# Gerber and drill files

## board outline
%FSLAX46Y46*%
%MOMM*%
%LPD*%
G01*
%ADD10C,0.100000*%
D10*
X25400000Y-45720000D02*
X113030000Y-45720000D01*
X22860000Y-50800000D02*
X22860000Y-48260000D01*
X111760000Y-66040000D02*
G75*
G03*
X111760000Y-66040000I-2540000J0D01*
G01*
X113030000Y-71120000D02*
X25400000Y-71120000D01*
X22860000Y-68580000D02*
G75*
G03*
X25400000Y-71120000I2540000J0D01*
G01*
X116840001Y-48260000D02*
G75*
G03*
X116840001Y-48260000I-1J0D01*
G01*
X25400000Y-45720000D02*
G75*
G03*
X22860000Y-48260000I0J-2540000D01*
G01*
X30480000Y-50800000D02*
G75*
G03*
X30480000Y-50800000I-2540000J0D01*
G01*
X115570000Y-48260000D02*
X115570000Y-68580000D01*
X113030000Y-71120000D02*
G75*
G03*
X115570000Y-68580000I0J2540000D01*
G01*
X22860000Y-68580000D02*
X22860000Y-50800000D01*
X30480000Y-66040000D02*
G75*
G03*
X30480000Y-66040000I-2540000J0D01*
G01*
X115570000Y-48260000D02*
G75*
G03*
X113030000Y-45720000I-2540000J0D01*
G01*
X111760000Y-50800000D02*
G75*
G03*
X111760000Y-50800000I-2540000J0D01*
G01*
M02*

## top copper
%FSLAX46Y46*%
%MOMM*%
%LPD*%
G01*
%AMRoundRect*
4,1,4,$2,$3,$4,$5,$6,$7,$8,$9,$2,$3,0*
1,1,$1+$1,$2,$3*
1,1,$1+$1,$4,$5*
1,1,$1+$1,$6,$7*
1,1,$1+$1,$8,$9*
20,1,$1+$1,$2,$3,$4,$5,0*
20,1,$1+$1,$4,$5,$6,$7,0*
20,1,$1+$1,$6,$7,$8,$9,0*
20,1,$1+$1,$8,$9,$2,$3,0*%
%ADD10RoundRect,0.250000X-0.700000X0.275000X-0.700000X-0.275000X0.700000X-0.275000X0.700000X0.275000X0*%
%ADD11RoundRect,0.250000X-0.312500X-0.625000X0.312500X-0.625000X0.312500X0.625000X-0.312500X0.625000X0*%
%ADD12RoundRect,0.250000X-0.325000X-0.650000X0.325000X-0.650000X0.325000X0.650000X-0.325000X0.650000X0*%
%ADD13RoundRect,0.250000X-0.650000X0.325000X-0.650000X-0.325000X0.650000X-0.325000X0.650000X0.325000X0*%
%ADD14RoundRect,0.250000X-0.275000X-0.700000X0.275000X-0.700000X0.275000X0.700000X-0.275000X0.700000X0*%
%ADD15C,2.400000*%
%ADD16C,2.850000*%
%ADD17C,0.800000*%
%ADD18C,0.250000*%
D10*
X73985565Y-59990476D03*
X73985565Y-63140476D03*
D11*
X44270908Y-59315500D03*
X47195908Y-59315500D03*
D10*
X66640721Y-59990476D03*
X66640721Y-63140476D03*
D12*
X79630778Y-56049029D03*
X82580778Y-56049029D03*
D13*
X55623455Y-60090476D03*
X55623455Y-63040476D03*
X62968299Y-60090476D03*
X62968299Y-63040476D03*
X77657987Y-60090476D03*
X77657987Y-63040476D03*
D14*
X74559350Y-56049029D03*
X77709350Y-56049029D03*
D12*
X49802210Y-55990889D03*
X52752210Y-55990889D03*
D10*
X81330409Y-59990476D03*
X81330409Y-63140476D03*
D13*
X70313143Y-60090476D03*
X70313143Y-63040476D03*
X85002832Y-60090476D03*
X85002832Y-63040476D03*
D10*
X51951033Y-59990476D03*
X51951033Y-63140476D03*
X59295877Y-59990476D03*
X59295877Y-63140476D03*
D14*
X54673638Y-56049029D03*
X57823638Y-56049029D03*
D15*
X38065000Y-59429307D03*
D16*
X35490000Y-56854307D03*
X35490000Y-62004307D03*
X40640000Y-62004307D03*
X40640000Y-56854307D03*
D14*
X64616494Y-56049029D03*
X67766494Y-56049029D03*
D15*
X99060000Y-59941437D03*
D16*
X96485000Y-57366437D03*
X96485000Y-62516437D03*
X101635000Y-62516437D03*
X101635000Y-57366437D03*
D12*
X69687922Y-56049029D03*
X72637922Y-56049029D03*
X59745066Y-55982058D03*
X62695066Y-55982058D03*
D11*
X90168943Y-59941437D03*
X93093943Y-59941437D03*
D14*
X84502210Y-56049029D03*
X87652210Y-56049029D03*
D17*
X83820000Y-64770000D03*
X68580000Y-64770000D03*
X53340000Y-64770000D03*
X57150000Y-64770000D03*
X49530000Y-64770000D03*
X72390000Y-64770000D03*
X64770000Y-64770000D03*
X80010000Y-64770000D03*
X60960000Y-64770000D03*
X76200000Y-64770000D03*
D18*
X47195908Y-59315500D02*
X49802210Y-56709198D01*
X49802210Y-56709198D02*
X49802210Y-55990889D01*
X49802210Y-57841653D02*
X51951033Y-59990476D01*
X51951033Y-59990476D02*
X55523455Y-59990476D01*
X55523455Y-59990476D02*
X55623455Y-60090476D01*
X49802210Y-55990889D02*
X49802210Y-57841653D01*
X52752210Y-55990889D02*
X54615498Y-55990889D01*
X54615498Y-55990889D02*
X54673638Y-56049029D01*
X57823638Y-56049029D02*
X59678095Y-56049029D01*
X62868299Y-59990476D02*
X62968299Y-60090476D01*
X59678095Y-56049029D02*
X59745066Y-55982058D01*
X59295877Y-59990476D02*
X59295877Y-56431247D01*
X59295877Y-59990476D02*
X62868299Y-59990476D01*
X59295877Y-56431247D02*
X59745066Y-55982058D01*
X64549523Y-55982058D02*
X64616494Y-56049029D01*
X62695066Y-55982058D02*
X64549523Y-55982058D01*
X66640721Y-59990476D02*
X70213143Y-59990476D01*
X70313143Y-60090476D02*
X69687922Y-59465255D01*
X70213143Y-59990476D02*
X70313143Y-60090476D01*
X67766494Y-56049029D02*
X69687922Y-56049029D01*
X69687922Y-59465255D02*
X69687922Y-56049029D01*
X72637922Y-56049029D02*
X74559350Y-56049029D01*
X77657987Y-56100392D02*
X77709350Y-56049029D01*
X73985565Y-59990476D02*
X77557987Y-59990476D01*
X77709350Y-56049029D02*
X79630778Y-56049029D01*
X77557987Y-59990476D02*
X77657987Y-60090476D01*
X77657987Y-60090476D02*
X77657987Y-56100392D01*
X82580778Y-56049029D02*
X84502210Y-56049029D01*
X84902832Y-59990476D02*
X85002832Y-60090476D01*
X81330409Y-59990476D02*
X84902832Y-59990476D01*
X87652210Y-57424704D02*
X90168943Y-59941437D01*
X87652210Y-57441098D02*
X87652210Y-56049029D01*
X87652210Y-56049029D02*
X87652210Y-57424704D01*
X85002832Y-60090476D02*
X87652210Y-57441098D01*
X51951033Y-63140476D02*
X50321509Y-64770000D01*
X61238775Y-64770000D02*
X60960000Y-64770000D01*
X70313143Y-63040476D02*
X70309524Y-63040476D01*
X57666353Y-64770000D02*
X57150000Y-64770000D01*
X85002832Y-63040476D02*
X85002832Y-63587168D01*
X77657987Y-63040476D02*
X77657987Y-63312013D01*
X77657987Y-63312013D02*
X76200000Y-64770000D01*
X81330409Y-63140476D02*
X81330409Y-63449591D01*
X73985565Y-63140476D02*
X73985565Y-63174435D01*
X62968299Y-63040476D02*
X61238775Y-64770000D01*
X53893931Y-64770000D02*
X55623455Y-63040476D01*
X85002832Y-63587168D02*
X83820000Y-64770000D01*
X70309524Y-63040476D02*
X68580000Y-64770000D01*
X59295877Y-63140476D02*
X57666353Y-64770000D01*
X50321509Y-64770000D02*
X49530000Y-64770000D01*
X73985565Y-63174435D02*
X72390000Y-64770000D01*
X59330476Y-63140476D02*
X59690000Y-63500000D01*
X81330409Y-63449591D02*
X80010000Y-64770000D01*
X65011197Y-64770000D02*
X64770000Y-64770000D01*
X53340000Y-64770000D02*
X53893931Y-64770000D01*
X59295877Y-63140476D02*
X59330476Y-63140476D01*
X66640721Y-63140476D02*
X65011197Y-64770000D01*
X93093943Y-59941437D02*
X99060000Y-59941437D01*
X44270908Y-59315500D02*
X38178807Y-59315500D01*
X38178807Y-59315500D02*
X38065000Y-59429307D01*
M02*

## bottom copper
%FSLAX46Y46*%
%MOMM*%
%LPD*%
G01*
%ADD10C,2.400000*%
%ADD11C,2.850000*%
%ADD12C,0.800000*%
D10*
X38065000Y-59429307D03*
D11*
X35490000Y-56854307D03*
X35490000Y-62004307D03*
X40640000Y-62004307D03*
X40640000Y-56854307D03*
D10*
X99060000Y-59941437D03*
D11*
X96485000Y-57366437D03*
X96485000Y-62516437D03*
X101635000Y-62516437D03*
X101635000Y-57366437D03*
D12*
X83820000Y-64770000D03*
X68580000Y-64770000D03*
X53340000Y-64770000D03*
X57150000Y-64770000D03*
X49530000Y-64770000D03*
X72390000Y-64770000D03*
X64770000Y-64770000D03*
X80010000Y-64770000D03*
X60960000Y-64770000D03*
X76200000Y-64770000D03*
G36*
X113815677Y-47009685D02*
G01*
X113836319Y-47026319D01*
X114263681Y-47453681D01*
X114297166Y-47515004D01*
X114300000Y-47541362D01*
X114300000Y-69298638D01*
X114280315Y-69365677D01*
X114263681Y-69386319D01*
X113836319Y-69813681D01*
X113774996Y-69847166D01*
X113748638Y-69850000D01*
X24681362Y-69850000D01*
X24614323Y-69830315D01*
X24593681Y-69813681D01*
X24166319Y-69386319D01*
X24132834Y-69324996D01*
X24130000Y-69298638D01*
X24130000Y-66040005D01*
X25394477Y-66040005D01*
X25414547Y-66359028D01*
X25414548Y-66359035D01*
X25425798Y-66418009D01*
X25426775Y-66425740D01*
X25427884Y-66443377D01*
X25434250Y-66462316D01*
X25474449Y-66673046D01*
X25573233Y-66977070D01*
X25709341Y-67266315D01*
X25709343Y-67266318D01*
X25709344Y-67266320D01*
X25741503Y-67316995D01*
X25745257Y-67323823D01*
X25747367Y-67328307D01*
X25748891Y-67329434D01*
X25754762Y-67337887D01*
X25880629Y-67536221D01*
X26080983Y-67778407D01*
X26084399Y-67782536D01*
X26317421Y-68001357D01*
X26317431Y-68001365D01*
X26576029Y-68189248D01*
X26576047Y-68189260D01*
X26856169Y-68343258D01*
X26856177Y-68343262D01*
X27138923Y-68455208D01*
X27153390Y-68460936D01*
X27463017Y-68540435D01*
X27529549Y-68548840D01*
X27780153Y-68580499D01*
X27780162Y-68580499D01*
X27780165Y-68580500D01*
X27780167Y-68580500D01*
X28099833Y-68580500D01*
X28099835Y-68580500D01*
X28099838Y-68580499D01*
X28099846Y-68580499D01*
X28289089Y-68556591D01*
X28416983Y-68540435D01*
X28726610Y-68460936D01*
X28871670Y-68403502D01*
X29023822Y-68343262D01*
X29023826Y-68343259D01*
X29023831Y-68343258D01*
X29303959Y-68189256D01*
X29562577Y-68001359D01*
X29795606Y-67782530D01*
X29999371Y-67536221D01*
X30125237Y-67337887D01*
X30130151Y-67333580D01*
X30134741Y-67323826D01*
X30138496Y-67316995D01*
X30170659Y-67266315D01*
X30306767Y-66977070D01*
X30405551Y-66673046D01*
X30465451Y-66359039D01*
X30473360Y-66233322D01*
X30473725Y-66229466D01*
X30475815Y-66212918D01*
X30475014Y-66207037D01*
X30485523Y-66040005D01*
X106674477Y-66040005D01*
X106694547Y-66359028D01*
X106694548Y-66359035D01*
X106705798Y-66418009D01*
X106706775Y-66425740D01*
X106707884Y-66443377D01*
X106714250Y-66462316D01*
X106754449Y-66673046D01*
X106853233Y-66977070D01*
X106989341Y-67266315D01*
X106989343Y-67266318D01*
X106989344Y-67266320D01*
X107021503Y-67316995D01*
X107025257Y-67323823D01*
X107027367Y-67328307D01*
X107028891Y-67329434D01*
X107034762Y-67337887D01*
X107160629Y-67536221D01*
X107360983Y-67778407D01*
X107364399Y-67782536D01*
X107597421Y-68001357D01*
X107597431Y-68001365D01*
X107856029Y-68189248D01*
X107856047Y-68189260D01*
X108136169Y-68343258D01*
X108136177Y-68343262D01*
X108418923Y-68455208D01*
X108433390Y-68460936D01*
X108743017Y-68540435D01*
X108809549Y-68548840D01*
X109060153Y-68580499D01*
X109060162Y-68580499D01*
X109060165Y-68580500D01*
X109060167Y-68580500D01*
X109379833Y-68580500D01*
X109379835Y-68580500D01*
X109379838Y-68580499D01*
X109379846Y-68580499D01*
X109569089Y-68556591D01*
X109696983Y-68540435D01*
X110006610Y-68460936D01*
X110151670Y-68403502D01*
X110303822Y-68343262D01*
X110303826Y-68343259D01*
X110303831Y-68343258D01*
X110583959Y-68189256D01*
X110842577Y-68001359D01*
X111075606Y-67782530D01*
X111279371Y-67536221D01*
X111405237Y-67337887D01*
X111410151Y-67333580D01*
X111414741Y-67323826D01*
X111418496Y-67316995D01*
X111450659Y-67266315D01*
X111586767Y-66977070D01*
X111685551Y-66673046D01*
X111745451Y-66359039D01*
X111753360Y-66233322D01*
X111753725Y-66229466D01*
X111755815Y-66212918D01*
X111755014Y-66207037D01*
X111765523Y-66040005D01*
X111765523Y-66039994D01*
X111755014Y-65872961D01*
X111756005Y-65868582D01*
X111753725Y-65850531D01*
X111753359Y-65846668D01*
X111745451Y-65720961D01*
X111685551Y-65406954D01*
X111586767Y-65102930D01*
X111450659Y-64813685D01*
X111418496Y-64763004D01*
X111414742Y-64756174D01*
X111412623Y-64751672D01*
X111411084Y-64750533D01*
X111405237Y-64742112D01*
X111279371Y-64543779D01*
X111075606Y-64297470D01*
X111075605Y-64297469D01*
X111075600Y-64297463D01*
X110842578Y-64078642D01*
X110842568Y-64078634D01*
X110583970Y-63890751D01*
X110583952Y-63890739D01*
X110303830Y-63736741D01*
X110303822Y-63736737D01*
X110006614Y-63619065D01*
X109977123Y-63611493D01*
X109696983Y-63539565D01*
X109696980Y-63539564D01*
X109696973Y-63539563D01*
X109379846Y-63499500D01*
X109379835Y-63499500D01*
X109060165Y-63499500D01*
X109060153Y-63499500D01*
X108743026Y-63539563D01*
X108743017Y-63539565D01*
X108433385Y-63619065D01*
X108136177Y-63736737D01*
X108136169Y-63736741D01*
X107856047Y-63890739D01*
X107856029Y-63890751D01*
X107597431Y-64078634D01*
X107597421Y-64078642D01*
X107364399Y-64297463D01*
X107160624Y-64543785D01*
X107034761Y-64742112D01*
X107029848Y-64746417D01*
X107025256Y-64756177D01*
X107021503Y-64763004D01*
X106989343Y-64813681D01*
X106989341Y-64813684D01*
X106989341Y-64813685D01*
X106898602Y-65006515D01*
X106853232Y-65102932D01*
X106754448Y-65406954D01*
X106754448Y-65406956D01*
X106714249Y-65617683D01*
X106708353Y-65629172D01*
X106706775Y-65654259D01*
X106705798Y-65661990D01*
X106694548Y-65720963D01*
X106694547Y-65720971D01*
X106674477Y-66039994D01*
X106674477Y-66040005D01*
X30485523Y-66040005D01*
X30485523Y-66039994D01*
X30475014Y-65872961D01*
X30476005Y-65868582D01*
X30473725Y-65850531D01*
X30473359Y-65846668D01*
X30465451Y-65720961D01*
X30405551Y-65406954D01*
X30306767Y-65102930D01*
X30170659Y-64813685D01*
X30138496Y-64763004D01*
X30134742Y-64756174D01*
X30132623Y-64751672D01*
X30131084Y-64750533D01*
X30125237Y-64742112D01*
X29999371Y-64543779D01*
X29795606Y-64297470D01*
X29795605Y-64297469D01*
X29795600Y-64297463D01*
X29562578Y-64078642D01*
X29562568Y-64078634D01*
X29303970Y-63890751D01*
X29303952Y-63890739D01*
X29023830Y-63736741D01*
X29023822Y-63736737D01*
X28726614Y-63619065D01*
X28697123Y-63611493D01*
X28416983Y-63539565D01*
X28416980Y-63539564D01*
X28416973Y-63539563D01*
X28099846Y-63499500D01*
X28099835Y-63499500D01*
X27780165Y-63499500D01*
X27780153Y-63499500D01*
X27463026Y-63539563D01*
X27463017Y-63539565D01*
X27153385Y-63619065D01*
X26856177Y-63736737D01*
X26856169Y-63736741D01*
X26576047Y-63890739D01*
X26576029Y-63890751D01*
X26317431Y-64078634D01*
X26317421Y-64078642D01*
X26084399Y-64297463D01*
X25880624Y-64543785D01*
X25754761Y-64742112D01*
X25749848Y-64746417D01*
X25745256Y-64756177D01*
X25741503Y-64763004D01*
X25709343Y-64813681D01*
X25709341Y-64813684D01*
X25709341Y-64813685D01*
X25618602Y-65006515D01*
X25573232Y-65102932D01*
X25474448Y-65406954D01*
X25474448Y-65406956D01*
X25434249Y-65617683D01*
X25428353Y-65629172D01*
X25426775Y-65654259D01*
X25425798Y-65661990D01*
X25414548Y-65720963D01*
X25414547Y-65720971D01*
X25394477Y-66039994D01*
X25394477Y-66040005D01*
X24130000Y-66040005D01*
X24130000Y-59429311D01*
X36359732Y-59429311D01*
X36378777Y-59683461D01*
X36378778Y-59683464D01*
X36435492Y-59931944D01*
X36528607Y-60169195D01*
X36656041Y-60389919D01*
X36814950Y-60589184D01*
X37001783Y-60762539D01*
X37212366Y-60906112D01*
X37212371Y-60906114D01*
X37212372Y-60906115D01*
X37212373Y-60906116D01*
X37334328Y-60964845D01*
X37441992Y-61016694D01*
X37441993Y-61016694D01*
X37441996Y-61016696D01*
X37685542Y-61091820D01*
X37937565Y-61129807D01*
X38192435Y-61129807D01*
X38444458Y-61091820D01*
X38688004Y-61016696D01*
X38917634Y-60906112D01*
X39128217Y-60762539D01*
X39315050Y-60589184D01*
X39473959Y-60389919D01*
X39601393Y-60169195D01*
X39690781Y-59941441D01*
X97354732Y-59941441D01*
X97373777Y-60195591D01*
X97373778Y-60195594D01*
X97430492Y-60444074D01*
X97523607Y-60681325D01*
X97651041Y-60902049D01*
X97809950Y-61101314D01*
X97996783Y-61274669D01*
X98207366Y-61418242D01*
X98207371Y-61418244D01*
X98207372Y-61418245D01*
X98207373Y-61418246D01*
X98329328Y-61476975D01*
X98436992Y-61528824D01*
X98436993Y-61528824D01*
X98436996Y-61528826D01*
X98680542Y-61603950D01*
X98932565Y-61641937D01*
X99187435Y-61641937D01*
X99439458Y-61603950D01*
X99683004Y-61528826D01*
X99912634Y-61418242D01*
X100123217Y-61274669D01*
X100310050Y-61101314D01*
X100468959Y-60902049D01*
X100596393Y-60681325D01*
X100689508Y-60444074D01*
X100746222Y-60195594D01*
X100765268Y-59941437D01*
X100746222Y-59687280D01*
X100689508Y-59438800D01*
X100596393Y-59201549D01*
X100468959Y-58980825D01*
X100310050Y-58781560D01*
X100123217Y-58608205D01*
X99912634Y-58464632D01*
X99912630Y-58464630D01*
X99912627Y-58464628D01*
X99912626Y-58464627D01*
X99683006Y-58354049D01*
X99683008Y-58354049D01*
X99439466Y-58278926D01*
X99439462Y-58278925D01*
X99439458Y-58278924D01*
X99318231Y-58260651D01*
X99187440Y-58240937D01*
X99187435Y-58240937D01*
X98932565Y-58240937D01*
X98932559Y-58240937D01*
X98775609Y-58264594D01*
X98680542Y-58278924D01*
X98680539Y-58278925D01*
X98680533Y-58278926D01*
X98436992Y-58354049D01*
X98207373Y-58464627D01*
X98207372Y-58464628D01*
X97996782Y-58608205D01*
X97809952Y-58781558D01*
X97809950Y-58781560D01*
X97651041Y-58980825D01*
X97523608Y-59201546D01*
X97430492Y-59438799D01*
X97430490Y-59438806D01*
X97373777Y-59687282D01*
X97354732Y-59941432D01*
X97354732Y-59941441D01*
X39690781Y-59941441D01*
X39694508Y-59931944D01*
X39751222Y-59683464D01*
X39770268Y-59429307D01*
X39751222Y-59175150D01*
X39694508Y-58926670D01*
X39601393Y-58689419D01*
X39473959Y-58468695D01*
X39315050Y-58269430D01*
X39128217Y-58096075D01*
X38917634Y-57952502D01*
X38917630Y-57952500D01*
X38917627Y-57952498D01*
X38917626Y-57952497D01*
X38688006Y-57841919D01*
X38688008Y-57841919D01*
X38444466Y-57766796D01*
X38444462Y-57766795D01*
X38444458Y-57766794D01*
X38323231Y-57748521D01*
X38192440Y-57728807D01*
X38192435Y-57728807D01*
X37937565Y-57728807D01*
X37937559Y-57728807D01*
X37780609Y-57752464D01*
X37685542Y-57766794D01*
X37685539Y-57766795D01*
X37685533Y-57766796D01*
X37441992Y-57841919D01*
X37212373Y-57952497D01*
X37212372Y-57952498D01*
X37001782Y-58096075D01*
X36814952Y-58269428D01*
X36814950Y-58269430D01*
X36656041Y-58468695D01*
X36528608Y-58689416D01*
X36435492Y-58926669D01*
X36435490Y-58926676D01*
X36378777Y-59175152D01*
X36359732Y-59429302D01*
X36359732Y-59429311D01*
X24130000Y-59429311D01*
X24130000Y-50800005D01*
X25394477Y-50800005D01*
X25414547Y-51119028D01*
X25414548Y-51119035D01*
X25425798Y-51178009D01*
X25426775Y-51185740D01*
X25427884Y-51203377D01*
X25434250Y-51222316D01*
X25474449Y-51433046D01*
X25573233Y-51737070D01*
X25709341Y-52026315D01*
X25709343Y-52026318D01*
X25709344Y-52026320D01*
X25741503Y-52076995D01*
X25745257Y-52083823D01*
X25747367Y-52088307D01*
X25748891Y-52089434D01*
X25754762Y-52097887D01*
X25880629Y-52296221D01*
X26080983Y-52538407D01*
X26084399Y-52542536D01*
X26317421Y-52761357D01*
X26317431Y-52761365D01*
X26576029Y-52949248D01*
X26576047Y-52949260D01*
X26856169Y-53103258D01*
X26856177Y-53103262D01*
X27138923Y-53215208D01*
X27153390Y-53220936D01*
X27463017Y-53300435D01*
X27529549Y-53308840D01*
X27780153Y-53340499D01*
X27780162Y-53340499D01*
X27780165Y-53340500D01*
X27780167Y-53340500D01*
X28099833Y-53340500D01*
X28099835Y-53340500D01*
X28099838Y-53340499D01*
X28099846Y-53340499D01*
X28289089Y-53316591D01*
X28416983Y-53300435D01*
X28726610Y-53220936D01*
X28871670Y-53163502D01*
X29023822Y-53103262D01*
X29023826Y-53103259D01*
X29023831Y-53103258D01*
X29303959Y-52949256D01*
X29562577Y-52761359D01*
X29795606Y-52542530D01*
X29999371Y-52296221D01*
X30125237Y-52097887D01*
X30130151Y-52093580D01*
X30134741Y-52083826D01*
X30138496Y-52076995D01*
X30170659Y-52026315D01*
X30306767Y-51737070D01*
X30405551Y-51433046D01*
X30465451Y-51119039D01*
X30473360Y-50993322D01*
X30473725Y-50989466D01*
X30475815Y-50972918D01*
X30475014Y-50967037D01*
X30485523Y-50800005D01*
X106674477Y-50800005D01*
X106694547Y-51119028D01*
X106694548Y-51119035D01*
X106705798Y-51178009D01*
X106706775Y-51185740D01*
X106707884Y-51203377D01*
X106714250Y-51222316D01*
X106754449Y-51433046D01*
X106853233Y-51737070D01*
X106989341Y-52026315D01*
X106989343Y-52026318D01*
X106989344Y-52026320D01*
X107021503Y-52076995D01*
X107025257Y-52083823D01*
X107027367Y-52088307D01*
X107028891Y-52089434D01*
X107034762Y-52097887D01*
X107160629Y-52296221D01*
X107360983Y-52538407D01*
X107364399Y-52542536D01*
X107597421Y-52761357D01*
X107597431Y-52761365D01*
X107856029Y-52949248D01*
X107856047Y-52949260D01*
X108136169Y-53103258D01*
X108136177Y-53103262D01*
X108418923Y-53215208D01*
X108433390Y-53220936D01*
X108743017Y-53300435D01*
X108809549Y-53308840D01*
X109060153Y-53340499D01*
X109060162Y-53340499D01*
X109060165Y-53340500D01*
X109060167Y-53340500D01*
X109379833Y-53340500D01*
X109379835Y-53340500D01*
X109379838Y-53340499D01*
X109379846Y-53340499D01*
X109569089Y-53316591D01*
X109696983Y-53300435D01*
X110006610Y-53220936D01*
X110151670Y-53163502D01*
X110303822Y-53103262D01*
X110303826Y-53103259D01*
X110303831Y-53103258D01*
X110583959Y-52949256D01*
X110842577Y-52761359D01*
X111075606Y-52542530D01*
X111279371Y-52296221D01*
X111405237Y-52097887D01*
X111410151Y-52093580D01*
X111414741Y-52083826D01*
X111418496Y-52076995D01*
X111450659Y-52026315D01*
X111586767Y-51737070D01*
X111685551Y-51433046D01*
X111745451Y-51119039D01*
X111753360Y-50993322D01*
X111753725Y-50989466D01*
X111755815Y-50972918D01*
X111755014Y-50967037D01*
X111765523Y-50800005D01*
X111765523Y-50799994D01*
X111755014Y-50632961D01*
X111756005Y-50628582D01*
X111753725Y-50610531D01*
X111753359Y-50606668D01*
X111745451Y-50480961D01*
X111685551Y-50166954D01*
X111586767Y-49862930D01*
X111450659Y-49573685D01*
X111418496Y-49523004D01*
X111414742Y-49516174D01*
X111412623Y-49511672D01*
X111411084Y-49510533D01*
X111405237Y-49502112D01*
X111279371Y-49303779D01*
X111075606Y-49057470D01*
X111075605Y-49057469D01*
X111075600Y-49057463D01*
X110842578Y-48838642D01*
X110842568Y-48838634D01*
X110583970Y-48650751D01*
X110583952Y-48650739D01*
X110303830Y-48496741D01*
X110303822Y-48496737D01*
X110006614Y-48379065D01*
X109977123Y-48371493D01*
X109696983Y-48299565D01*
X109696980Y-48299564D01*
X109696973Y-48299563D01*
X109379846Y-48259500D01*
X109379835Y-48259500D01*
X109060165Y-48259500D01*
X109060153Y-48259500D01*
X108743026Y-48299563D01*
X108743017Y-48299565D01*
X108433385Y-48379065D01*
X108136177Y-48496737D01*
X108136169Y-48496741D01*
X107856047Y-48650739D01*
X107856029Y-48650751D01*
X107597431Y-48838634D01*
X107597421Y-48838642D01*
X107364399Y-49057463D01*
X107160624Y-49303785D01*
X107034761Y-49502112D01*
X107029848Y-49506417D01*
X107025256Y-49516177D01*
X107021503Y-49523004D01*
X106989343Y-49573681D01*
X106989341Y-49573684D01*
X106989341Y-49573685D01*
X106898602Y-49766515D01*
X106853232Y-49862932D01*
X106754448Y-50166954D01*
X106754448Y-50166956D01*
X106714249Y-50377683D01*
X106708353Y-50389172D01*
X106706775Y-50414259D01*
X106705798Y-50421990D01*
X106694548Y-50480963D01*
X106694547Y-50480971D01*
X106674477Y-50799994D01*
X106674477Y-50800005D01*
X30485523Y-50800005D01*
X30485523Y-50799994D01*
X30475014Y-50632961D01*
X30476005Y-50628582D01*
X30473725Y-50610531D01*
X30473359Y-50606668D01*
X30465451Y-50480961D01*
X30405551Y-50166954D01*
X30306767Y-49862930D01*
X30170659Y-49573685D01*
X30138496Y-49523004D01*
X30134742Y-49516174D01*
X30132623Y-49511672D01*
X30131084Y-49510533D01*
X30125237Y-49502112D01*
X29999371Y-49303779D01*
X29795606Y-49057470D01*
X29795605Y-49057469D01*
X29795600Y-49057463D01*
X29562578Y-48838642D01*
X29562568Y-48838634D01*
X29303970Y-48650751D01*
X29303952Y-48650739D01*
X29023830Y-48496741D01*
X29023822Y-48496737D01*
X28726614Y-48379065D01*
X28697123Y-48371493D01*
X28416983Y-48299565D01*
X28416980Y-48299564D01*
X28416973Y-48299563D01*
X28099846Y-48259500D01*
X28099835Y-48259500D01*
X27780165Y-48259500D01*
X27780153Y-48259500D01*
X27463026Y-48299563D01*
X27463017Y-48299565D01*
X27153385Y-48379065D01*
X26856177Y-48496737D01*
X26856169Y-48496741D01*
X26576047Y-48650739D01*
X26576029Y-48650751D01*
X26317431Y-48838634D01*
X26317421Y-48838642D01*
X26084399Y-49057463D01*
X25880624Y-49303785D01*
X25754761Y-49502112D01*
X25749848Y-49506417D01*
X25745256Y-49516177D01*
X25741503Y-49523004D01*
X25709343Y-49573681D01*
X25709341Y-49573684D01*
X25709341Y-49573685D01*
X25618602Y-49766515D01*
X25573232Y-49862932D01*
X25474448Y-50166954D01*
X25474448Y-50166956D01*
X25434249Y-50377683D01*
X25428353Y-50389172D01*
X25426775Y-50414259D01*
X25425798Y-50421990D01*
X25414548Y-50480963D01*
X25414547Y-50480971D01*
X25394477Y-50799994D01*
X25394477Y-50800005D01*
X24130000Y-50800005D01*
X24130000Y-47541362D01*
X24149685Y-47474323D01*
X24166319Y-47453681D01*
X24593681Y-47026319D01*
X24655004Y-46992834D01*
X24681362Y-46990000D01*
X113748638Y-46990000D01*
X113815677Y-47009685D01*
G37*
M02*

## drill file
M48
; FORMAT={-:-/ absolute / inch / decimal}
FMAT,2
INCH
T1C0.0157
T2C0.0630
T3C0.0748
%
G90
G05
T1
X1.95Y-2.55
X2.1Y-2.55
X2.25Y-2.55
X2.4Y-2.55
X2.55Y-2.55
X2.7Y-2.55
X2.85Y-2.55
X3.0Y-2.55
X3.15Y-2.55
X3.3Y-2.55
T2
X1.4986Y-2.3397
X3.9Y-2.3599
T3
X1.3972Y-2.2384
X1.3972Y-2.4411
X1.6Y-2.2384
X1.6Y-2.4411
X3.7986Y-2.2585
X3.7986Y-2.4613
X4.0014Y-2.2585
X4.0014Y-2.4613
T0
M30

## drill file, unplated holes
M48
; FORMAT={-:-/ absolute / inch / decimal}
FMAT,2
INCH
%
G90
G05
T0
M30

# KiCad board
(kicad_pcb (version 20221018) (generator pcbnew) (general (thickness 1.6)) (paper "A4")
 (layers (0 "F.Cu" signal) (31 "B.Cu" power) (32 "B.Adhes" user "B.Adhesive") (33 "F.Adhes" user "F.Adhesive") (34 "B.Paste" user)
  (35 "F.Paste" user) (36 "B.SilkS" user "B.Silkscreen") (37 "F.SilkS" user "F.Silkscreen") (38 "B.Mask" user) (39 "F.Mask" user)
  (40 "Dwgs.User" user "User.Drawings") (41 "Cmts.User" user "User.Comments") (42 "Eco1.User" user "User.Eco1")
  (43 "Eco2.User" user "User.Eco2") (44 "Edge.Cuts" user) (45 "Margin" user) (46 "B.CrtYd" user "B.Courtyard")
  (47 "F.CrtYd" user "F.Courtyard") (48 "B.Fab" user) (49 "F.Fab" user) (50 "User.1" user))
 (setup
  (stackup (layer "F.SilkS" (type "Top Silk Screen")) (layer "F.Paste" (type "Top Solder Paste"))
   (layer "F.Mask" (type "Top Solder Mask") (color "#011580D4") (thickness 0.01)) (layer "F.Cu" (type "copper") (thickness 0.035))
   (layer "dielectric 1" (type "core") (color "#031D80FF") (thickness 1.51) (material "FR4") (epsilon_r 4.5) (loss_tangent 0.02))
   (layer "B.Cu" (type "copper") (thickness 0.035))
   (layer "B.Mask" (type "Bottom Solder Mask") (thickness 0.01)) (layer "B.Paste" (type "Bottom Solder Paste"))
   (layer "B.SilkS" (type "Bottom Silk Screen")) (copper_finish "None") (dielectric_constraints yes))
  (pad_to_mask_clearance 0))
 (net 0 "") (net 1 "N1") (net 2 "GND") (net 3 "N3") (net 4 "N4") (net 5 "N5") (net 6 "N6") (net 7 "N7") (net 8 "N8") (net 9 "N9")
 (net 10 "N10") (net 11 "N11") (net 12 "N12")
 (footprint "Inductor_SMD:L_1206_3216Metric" (layer "F.Cu") (at 73.985565 61.565476 -90)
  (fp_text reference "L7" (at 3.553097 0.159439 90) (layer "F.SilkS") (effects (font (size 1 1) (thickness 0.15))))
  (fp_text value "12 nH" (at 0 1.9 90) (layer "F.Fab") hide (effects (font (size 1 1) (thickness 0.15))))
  (pad "1" smd roundrect (at -1.575 0 270) (size 1.05 1.9) (layers "F.Cu" "F.Paste" "F.Mask") (roundrect_rratio 0.2380952381) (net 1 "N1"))
  (pad "2" smd roundrect (at 1.575 0 270) (size 1.05 1.9) (layers "F.Cu" "F.Paste" "F.Mask") (roundrect_rratio 0.2380952381) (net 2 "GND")))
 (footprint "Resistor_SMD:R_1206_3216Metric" (layer "F.Cu") (at 45.733408 59.3155)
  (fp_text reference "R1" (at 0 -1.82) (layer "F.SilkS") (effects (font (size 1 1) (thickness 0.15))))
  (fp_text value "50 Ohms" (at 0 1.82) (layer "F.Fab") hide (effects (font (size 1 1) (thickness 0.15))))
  (pad "1" smd roundrect (at -1.4625 0) (size 1.125 1.75) (layers "F.Cu" "F.Paste" "F.Mask") (roundrect_rratio 0.2222222222) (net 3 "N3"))
  (pad "2" smd roundrect (at 1.4625 0) (size 1.125 1.75) (layers "F.Cu" "F.Paste" "F.Mask") (roundrect_rratio 0.2222222222) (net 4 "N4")))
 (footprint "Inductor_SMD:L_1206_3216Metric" (layer "F.Cu") (at 66.640721 61.565476 -90)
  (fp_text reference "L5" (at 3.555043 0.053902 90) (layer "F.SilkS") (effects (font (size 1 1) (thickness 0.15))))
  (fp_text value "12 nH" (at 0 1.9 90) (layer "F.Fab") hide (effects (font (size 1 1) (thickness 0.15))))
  (pad "1" smd roundrect (at -1.575 0 270) (size 1.05 1.9) (layers "F.Cu" "F.Paste" "F.Mask") (roundrect_rratio 0.2380952381) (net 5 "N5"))
  (pad "2" smd roundrect (at 1.575 0 270) (size 1.05 1.9) (layers "F.Cu" "F.Paste" "F.Mask") (roundrect_rratio 0.2380952381) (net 2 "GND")))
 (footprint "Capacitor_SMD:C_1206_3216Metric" (layer "F.Cu") (at 81.105778 56.049029)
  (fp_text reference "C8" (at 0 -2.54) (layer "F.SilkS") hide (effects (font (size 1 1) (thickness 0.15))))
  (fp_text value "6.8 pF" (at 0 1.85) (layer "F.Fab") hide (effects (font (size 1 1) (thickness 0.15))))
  (pad "1" smd roundrect (at -1.475 0) (size 1.15 1.8) (layers "F.Cu" "F.Paste" "F.Mask") (roundrect_rratio 0.2173913043) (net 1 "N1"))
  (pad "2" smd roundrect (at 1.475 0) (size 1.15 1.8) (layers "F.Cu" "F.Paste" "F.Mask") (roundrect_rratio 0.2173913043) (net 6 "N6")))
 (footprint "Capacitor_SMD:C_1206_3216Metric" (layer "F.Cu") (at 55.623455 61.565476 -90)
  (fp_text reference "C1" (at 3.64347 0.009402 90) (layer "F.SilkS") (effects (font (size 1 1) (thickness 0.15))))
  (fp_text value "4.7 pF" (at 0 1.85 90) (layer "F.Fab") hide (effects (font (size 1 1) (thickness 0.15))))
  (pad "1" smd roundrect (at -1.475 0 270) (size 1.15 1.8) (layers "F.Cu" "F.Paste" "F.Mask") (roundrect_rratio 0.2173913043) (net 4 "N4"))
  (pad "2" smd roundrect (at 1.475 0 270) (size 1.15 1.8) (layers "F.Cu" "F.Paste" "F.Mask") (roundrect_rratio 0.2173913043) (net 2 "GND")))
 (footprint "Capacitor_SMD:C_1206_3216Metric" (layer "F.Cu") (at 62.968299 61.565476 -90)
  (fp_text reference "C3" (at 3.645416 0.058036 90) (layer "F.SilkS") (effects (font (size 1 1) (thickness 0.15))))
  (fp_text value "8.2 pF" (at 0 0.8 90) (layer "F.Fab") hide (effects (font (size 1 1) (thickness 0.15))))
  (pad "1" smd roundrect (at -1.475 0 270) (size 1.15 1.8) (layers "F.Cu" "F.Paste" "F.Mask") (roundrect_rratio 0.2173913043) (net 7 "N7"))
  (pad "2" smd roundrect (at 1.475 0 270) (size 1.15 1.8) (layers "F.Cu" "F.Paste" "F.Mask") (roundrect_rratio 0.2173913043) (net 2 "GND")))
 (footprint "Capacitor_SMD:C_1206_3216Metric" (layer "F.Cu") (at 77.657987 61.565476 -90)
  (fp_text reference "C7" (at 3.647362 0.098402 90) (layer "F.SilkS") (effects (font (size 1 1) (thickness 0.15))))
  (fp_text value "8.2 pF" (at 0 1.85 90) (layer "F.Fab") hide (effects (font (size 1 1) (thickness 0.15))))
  (pad "1" smd roundrect (at -1.475 0 270) (size 1.15 1.8) (layers "F.Cu" "F.Paste" "F.Mask") (roundrect_rratio 0.2173913043) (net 1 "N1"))
  (pad "2" smd roundrect (at 1.475 0 270) (size 1.15 1.8) (layers "F.Cu" "F.Paste" "F.Mask") (roundrect_rratio 0.2173913043) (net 2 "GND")))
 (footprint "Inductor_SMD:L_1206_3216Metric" (layer "F.Cu") (at 76.13435 56.049029)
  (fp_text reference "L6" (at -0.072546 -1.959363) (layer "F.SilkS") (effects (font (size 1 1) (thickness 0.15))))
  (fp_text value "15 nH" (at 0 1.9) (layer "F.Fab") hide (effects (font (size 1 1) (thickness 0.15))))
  (pad "1" smd roundrect (at -1.575 0) (size 1.05 1.9) (layers "F.Cu" "F.Paste" "F.Mask") (roundrect_rratio 0.2380952381) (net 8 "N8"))
  (pad "2" smd roundrect (at 1.575 0) (size 1.05 1.9) (layers "F.Cu" "F.Paste" "F.Mask") (roundrect_rratio 0.2380952381) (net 1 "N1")))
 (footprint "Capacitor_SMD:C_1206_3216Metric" (layer "F.Cu") (at 51.27721 55.990889)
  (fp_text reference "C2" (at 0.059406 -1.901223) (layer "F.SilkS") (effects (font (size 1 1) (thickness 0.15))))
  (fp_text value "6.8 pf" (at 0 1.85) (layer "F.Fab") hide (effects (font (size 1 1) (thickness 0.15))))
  (pad "1" smd roundrect (at -1.475 0) (size 1.15 1.8) (layers "F.Cu" "F.Paste" "F.Mask") (roundrect_rratio 0.2173913043) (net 4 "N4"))
  (pad "2" smd roundrect (at 1.475 0) (size 1.15 1.8) (layers "F.Cu" "F.Paste" "F.Mask") (roundrect_rratio 0.2173913043) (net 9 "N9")))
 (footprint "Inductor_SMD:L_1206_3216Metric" (layer "F.Cu") (at 81.330409 61.565476 -90)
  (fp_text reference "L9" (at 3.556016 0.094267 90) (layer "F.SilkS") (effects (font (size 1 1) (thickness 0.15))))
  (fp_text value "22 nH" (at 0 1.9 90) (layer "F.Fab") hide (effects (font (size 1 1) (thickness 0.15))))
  (pad "1" smd roundrect (at -1.575 0 270) (size 1.05 1.9) (layers "F.Cu" "F.Paste" "F.Mask") (roundrect_rratio 0.2380952381) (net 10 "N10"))
  (pad "2" smd roundrect (at 1.575 0 270) (size 1.05 1.9) (layers "F.Cu" "F.Paste" "F.Mask") (roundrect_rratio 0.2380952381) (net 2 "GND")))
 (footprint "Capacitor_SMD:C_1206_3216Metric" (layer "F.Cu") (at 70.313143 61.565476 -90)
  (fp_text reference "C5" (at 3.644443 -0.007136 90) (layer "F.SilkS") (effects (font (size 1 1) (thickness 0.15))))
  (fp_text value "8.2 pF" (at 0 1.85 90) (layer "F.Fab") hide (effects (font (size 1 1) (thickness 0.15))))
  (pad "1" smd roundrect (at -1.475 0 270) (size 1.15 1.8) (layers "F.Cu" "F.Paste" "F.Mask") (roundrect_rratio 0.2173913043) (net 5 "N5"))
  (pad "2" smd roundrect (at 1.475 0 270) (size 1.15 1.8) (layers "F.Cu" "F.Paste" "F.Mask") (roundrect_rratio 0.2173913043) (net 2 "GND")))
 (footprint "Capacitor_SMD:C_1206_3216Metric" (layer "F.Cu") (at 85.002832 61.565476 -90)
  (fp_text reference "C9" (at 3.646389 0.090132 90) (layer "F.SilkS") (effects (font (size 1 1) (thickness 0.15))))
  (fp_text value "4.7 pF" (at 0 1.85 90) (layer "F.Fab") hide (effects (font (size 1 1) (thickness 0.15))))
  (pad "1" smd roundrect (at -1.475 0 270) (size 1.15 1.8) (layers "F.Cu" "F.Paste" "F.Mask") (roundrect_rratio 0.2173913043) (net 10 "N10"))
  (pad "2" smd roundrect (at 1.475 0 270) (size 1.15 1.8) (layers "F.Cu" "F.Paste" "F.Mask") (roundrect_rratio 0.2173913043) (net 2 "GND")))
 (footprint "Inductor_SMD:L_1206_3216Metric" (layer "F.Cu") (at 51.951033 61.565476 -90)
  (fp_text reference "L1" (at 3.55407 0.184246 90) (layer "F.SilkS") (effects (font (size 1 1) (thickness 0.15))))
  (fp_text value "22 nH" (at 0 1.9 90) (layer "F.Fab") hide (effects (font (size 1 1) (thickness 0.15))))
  (pad "1" smd roundrect (at -1.575 0 270) (size 1.05 1.9) (layers "F.Cu" "F.Paste" "F.Mask") (roundrect_rratio 0.2380952381) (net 4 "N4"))
  (pad "2" smd roundrect (at 1.575 0 270) (size 1.05 1.9) (layers "F.Cu" "F.Paste" "F.Mask") (roundrect_rratio 0.2380952381) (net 2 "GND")))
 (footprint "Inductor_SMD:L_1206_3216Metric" (layer "F.Cu") (at 59.295877 61.565476 -90)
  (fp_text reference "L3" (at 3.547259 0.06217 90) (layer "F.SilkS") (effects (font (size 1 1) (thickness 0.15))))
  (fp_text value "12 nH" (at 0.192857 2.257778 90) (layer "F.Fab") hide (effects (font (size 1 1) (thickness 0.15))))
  (pad "1" smd roundrect (at -1.575 0 270) (size 1.05 1.9) (layers "F.Cu" "F.Paste" "F.Mask") (roundrect_rratio 0.2380952381) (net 7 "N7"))
  (pad "2" smd roundrect (at 1.575 0 270) (size 1.05 1.9) (layers "F.Cu" "F.Paste" "F.Mask") (roundrect_rratio 0.2380952381) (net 2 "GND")))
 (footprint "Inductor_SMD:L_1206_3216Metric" (layer "F.Cu") (at 56.248638 56.049029)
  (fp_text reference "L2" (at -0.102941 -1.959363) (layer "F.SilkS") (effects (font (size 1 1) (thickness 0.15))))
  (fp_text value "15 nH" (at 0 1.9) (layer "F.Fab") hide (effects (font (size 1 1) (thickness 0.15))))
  (pad "1" smd roundrect (at -1.575 0) (size 1.05 1.9) (layers "F.Cu" "F.Paste" "F.Mask") (roundrect_rratio 0.2380952381) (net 9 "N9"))
  (pad "2" smd roundrect (at 1.575 0) (size 1.05 1.9) (layers "F.Cu" "F.Paste" "F.Mask") (roundrect_rratio 0.2380952381) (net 7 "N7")))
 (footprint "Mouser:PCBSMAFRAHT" (layer "F.Cu") (at 38.065 59.429307)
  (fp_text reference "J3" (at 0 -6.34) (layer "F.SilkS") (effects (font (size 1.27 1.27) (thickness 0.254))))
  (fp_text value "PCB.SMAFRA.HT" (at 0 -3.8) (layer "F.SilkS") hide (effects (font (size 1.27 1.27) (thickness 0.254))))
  (pad "1" thru_hole circle (at 0 0) (size 2.4 2.4) (drill 1.6) (layers "*.Cu" "*.Mask") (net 3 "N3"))
  (pad "2" thru_hole circle (at -2.575 -2.575) (size 2.85 2.85) (drill 1.9) (layers "*.Cu" "*.Mask") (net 2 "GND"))
  (pad "3" thru_hole circle (at -2.575 2.575) (size 2.85 2.85) (drill 1.9) (layers "*.Cu" "*.Mask") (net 2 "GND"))
  (pad "4" thru_hole circle (at 2.575 2.575) (size 2.85 2.85) (drill 1.9) (layers "*.Cu" "*.Mask") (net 2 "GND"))
  (pad "5" thru_hole circle (at 2.575 -2.575) (size 2.85 2.85) (drill 1.9) (layers "*.Cu" "*.Mask") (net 2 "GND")))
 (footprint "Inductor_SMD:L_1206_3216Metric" (layer "F.Cu") (at 66.191494 56.049029)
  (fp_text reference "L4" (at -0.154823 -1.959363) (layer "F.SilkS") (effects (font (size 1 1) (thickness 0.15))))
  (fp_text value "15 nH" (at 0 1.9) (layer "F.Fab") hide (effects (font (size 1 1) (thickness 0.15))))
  (pad "1" smd roundrect (at -1.575 0) (size 1.05 1.9) (layers "F.Cu" "F.Paste" "F.Mask") (roundrect_rratio 0.2380952381) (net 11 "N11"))
  (pad "2" smd roundrect (at 1.575 0) (size 1.05 1.9) (layers "F.Cu" "F.Paste" "F.Mask") (roundrect_rratio 0.2380952381) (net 5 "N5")))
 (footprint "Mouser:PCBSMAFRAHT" (layer "F.Cu") (at 99.06 59.941437)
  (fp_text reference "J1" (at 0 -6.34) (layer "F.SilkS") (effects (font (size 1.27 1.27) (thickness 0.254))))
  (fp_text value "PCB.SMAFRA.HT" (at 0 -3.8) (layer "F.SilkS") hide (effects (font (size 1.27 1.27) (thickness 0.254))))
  (pad "1" thru_hole circle (at 0 0) (size 2.4 2.4) (drill 1.6) (layers "*.Cu" "*.Mask") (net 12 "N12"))
  (pad "2" thru_hole circle (at -2.575 -2.575) (size 2.85 2.85) (drill 1.9) (layers "*.Cu" "*.Mask") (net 2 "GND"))
  (pad "3" thru_hole circle (at -2.575 2.575) (size 2.85 2.85) (drill 1.9) (layers "*.Cu" "*.Mask") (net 2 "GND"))
  (pad "4" thru_hole circle (at 2.575 2.575) (size 2.85 2.85) (drill 1.9) (layers "*.Cu" "*.Mask") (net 2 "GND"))
  (pad "5" thru_hole circle (at 2.575 -2.575) (size 2.85 2.85) (drill 1.9) (layers "*.Cu" "*.Mask") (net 2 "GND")))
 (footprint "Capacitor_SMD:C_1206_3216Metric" (layer "F.Cu") (at 71.162922 56.049029)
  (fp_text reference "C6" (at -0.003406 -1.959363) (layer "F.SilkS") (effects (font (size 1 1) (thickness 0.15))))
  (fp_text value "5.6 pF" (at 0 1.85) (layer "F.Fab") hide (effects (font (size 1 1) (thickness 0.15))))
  (pad "1" smd roundrect (at -1.475 0) (size 1.15 1.8) (layers "F.Cu" "F.Paste" "F.Mask") (roundrect_rratio 0.2173913043) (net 5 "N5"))
  (pad "2" smd roundrect (at 1.475 0) (size 1.15 1.8) (layers "F.Cu" "F.Paste" "F.Mask") (roundrect_rratio 0.2173913043) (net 8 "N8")))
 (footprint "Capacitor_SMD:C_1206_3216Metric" (layer "F.Cu") (at 61.220066 55.982058)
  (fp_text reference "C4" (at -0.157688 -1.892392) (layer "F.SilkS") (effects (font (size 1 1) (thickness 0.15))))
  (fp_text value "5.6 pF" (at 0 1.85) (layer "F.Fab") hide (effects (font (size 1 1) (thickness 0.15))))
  (pad "1" smd roundrect (at -1.475 0) (size 1.15 1.8) (layers "F.Cu" "F.Paste" "F.Mask") (roundrect_rratio 0.2173913043) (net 7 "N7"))
  (pad "2" smd roundrect (at 1.475 0) (size 1.15 1.8) (layers "F.Cu" "F.Paste" "F.Mask") (roundrect_rratio 0.2173913043) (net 11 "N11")))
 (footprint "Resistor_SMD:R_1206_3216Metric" (layer "F.Cu") (at 91.631443 59.941437)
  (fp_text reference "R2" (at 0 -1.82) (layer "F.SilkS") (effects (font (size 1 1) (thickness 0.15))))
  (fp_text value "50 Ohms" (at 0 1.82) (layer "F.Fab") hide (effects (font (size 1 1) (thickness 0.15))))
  (pad "1" smd roundrect (at -1.4625 0) (size 1.125 1.75) (layers "F.Cu" "F.Paste" "F.Mask") (roundrect_rratio 0.2222222222) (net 10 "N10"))
  (pad "2" smd roundrect (at 1.4625 0) (size 1.125 1.75) (layers "F.Cu" "F.Paste" "F.Mask") (roundrect_rratio 0.2222222222) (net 12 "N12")))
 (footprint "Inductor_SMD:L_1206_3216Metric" (layer "F.Cu") (at 86.07721 56.049029)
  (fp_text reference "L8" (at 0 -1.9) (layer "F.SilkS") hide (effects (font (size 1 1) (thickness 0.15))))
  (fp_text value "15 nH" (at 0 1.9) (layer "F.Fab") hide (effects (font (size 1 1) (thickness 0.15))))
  (pad "1" smd roundrect (at -1.575 0) (size 1.05 1.9) (layers "F.Cu" "F.Paste" "F.Mask") (roundrect_rratio 0.2380952381) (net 6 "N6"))
  (pad "2" smd roundrect (at 1.575 0) (size 1.05 1.9) (layers "F.Cu" "F.Paste" "F.Mask") (roundrect_rratio 0.2380952381) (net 10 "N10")))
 (gr_line (start 25.4 45.72) (end 113.03 45.72) (stroke (width 0.1) (type default)) (layer "Edge.Cuts"))
 (gr_line (start 22.86 50.8) (end 22.86 48.26) (stroke (width 0.1) (type default)) (layer "Edge.Cuts"))
 (gr_circle (center 109.22 66.04) (end 111.76 66.04) (stroke (width 0.1) (type default)) (fill none) (layer "Edge.Cuts"))
 (gr_line (start 113.03 71.12) (end 25.4 71.12) (stroke (width 0.1) (type default)) (layer "Edge.Cuts"))
 (gr_arc (start 25.4 71.12) (mid 23.603949 70.376051) (end 22.86 68.58) (stroke (width 0.1) (type default)) (layer "Edge.Cuts"))
 (gr_circle (center 116.84 48.26) (end 116.84 48.26) (stroke (width 0.1) (type default)) (fill none) (layer "Edge.Cuts"))
 (gr_arc (start 22.86 48.26) (mid 23.603949 46.463949) (end 25.4 45.72) (stroke (width 0.1) (type default)) (layer "Edge.Cuts"))
 (gr_circle (center 27.94 50.8) (end 27.94 48.26) (stroke (width 0.1) (type default)) (fill none) (layer "Edge.Cuts"))
 (gr_line (start 115.57 48.26) (end 115.57 68.58) (stroke (width 0.1) (type default)) (layer "Edge.Cuts"))
 (gr_arc (start 115.57 68.58) (mid 114.826051 70.376051) (end 113.03 71.12) (stroke (width 0.1) (type default)) (layer "Edge.Cuts"))
 (gr_line (start 22.86 68.58) (end 22.86 50.8) (stroke (width 0.1) (type default)) (layer "Edge.Cuts"))
 (gr_circle (center 27.94 66.04) (end 25.4 66.04) (stroke (width 0.1) (type default)) (fill none) (layer "Edge.Cuts"))
 (gr_arc (start 113.03 45.72) (mid 114.826051 46.463949) (end 115.57 48.26) (stroke (width 0.1) (type default)) (layer "Edge.Cuts"))
 (gr_circle (center 109.22 50.8) (end 106.68 50.8) (stroke (width 0.1) (type default)) (fill none) (layer "Edge.Cuts"))
 (segment (start 47.195908 59.3155) (end 49.80221 56.709198) (width 0.25) (layer "F.Cu") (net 4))
 (segment (start 49.80221 56.709198) (end 49.80221 55.990889) (width 0.25) (layer "F.Cu") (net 4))
 (segment (start 49.80221 57.841653) (end 51.951033 59.990476) (width 0.25) (layer "F.Cu") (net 4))
 (segment (start 51.951033 59.990476) (end 55.523455 59.990476) (width 0.25) (layer "F.Cu") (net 4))
 (segment (start 55.523455 59.990476) (end 55.623455 60.090476) (width 0.25) (layer "F.Cu") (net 4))
 (segment (start 49.80221 55.990889) (end 49.80221 57.841653) (width 0.25) (layer "F.Cu") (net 4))
 (segment (start 52.75221 55.990889) (end 54.615498 55.990889) (width 0.25) (layer "F.Cu") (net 9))
 (segment (start 54.615498 55.990889) (end 54.673638 56.049029) (width 0.25) (layer "F.Cu") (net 9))
 (segment (start 57.823638 56.049029) (end 59.678095 56.049029) (width 0.25) (layer "F.Cu") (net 7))
 (segment (start 62.868299 59.990476) (end 62.968299 60.090476) (width 0.25) (layer "F.Cu") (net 7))
 (segment (start 59.678095 56.049029) (end 59.745066 55.982058) (width 0.25) (layer "F.Cu") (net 7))
 (segment (start 59.295877 59.990476) (end 59.295877 56.431247) (width 0.25) (layer "F.Cu") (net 7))
 (segment (start 59.295877 59.990476) (end 62.868299 59.990476) (width 0.25) (layer "F.Cu") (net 7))
 (segment (start 59.295877 56.431247) (end 59.745066 55.982058) (width 0.25) (layer "F.Cu") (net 7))
 (segment (start 64.549523 55.982058) (end 64.616494 56.049029) (width 0.25) (layer "F.Cu") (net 11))
 (segment (start 62.695066 55.982058) (end 64.549523 55.982058) (width 0.25) (layer "F.Cu") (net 11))
 (segment (start 66.640721 59.990476) (end 70.213143 59.990476) (width 0.25) (layer "F.Cu") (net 5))
 (segment (start 70.313143 60.090476) (end 69.687922 59.465255) (width 0.25) (layer "F.Cu") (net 5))
 (segment (start 70.213143 59.990476) (end 70.313143 60.090476) (width 0.25) (layer "F.Cu") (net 5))
 (segment (start 67.766494 56.049029) (end 69.687922 56.049029) (width 0.25) (layer "F.Cu") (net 5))
 (segment (start 69.687922 59.465255) (end 69.687922 56.049029) (width 0.25) (layer "F.Cu") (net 5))
 (segment (start 72.637922 56.049029) (end 74.55935 56.049029) (width 0.25) (layer "F.Cu") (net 8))
 (segment (start 77.657987 56.100392) (end 77.70935 56.049029) (width 0.25) (layer "F.Cu") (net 1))
 (segment (start 73.985565 59.990476) (end 77.557987 59.990476) (width 0.25) (layer "F.Cu") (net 1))
 (segment (start 77.70935 56.049029) (end 79.630778 56.049029) (width 0.25) (layer "F.Cu") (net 1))
 (segment (start 77.557987 59.990476) (end 77.657987 60.090476) (width 0.25) (layer "F.Cu") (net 1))
 (segment (start 77.657987 60.090476) (end 77.657987 56.100392) (width 0.25) (layer "F.Cu") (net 1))
 (segment (start 82.580778 56.049029) (end 84.50221 56.049029) (width 0.25) (layer "F.Cu") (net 6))
 (segment (start 84.902832 59.990476) (end 85.002832 60.090476) (width 0.25) (layer "F.Cu") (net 10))
 (segment (start 81.330409 59.990476) (end 84.902832 59.990476) (width 0.25) (layer "F.Cu") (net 10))
 (segment (start 87.65221 57.424704) (end 90.168943 59.941437) (width 0.25) (layer "F.Cu") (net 10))
 (segment (start 87.65221 57.441098) (end 87.65221 56.049029) (width 0.25) (layer "F.Cu") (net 10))
 (segment (start 87.65221 56.049029) (end 87.65221 57.424704) (width 0.25) (layer "F.Cu") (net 10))
 (segment (start 85.002832 60.090476) (end 87.65221 57.441098) (width 0.25) (layer "F.Cu") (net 10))
 (segment (start 51.951033 63.140476) (end 50.321509 64.77) (width 0.25) (layer "F.Cu") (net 2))
 (segment (start 61.238775 64.77) (end 60.96 64.77) (width 0.25) (layer "F.Cu") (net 2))
 (segment (start 70.313143 63.040476) (end 70.309524 63.040476) (width 0.25) (layer "F.Cu") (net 2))
 (segment (start 57.666353 64.77) (end 57.15 64.77) (width 0.25) (layer "F.Cu") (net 2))
 (segment (start 85.002832 63.040476) (end 85.002832 63.587168) (width 0.25) (layer "F.Cu") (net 2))
 (segment (start 77.657987 63.040476) (end 77.657987 63.312013) (width 0.25) (layer "F.Cu") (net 2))
 (segment (start 77.657987 63.312013) (end 76.2 64.77) (width 0.25) (layer "F.Cu") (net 2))
 (segment (start 81.330409 63.140476) (end 81.330409 63.449591) (width 0.25) (layer "F.Cu") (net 2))
 (segment (start 73.985565 63.140476) (end 73.985565 63.174435) (width 0.25) (layer "F.Cu") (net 2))
 (segment (start 62.968299 63.040476) (end 61.238775 64.77) (width 0.25) (layer "F.Cu") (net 2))
 (segment (start 53.893931 64.77) (end 55.623455 63.040476) (width 0.25) (layer "F.Cu") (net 2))
 (segment (start 85.002832 63.587168) (end 83.82 64.77) (width 0.25) (layer "F.Cu") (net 2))
 (segment (start 70.309524 63.040476) (end 68.58 64.77) (width 0.25) (layer "F.Cu") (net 2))
 (segment (start 59.295877 63.140476) (end 57.666353 64.77) (width 0.25) (layer "F.Cu") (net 2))
 (segment (start 50.321509 64.77) (end 49.53 64.77) (width 0.25) (layer "F.Cu") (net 2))
 (segment (start 73.985565 63.174435) (end 72.39 64.77) (width 0.25) (layer "F.Cu") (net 2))
 (segment (start 59.330476 63.140476) (end 59.69 63.5) (width 0.25) (layer "F.Cu") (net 2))
 (segment (start 81.330409 63.449591) (end 80.01 64.77) (width 0.25) (layer "F.Cu") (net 2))
 (segment (start 65.011197 64.77) (end 64.77 64.77) (width 0.25) (layer "F.Cu") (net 2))
 (segment (start 53.34 64.77) (end 53.893931 64.77) (width 0.25) (layer "F.Cu") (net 2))
 (segment (start 59.295877 63.140476) (end 59.330476 63.140476) (width 0.25) (layer "F.Cu") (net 2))
 (segment (start 66.640721 63.140476) (end 65.011197 64.77) (width 0.25) (layer "F.Cu") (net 2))
 (via (at 83.82 64.77) (size 0.8) (drill 0.4) (layers "F.Cu" "B.Cu") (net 2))
 (via (at 68.58 64.77) (size 0.8) (drill 0.4) (layers "F.Cu" "B.Cu") (free) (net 2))
 (via (at 53.34 64.77) (size 0.8) (drill 0.4) (layers "F.Cu" "B.Cu") (free) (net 2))
 (via (at 57.15 64.77) (size 0.8) (drill 0.4) (layers "F.Cu" "B.Cu") (free) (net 2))
 (via (at 49.53 64.77) (size 0.8) (drill 0.4) (layers "F.Cu" "B.Cu") (free) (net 2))
 (via (at 72.39 64.77) (size 0.8) (drill 0.4) (layers "F.Cu" "B.Cu") (free) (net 2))
 (via (at 64.77 64.77) (size 0.8) (drill 0.4) (layers "F.Cu" "B.Cu") (free) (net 2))
 (via (at 80.01 64.77) (size 0.8) (drill 0.4) (layers "F.Cu" "B.Cu") (free) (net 2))
 (via (at 60.96 64.77) (size 0.8) (drill 0.4) (layers "F.Cu" "B.Cu") (free) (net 2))
 (via (at 76.2 64.77) (size 0.8) (drill 0.4) (layers "F.Cu" "B.Cu") (free) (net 2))
 (segment (start 93.093943 59.941437) (end 99.06 59.941437) (width 0.25) (layer "F.Cu") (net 12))
 (segment (start 44.270908 59.3155) (end 38.178807 59.3155) (width 0.25) (layer "F.Cu") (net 3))
 (segment (start 38.178807 59.3155) (end 38.065 59.429307) (width 0.25) (layer "F.Cu") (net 3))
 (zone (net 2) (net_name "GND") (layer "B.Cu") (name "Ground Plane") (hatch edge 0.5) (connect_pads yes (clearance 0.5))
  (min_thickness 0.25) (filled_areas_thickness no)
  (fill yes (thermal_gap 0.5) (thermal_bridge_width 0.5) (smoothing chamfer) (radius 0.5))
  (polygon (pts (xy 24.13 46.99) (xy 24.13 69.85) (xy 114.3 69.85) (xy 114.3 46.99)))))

